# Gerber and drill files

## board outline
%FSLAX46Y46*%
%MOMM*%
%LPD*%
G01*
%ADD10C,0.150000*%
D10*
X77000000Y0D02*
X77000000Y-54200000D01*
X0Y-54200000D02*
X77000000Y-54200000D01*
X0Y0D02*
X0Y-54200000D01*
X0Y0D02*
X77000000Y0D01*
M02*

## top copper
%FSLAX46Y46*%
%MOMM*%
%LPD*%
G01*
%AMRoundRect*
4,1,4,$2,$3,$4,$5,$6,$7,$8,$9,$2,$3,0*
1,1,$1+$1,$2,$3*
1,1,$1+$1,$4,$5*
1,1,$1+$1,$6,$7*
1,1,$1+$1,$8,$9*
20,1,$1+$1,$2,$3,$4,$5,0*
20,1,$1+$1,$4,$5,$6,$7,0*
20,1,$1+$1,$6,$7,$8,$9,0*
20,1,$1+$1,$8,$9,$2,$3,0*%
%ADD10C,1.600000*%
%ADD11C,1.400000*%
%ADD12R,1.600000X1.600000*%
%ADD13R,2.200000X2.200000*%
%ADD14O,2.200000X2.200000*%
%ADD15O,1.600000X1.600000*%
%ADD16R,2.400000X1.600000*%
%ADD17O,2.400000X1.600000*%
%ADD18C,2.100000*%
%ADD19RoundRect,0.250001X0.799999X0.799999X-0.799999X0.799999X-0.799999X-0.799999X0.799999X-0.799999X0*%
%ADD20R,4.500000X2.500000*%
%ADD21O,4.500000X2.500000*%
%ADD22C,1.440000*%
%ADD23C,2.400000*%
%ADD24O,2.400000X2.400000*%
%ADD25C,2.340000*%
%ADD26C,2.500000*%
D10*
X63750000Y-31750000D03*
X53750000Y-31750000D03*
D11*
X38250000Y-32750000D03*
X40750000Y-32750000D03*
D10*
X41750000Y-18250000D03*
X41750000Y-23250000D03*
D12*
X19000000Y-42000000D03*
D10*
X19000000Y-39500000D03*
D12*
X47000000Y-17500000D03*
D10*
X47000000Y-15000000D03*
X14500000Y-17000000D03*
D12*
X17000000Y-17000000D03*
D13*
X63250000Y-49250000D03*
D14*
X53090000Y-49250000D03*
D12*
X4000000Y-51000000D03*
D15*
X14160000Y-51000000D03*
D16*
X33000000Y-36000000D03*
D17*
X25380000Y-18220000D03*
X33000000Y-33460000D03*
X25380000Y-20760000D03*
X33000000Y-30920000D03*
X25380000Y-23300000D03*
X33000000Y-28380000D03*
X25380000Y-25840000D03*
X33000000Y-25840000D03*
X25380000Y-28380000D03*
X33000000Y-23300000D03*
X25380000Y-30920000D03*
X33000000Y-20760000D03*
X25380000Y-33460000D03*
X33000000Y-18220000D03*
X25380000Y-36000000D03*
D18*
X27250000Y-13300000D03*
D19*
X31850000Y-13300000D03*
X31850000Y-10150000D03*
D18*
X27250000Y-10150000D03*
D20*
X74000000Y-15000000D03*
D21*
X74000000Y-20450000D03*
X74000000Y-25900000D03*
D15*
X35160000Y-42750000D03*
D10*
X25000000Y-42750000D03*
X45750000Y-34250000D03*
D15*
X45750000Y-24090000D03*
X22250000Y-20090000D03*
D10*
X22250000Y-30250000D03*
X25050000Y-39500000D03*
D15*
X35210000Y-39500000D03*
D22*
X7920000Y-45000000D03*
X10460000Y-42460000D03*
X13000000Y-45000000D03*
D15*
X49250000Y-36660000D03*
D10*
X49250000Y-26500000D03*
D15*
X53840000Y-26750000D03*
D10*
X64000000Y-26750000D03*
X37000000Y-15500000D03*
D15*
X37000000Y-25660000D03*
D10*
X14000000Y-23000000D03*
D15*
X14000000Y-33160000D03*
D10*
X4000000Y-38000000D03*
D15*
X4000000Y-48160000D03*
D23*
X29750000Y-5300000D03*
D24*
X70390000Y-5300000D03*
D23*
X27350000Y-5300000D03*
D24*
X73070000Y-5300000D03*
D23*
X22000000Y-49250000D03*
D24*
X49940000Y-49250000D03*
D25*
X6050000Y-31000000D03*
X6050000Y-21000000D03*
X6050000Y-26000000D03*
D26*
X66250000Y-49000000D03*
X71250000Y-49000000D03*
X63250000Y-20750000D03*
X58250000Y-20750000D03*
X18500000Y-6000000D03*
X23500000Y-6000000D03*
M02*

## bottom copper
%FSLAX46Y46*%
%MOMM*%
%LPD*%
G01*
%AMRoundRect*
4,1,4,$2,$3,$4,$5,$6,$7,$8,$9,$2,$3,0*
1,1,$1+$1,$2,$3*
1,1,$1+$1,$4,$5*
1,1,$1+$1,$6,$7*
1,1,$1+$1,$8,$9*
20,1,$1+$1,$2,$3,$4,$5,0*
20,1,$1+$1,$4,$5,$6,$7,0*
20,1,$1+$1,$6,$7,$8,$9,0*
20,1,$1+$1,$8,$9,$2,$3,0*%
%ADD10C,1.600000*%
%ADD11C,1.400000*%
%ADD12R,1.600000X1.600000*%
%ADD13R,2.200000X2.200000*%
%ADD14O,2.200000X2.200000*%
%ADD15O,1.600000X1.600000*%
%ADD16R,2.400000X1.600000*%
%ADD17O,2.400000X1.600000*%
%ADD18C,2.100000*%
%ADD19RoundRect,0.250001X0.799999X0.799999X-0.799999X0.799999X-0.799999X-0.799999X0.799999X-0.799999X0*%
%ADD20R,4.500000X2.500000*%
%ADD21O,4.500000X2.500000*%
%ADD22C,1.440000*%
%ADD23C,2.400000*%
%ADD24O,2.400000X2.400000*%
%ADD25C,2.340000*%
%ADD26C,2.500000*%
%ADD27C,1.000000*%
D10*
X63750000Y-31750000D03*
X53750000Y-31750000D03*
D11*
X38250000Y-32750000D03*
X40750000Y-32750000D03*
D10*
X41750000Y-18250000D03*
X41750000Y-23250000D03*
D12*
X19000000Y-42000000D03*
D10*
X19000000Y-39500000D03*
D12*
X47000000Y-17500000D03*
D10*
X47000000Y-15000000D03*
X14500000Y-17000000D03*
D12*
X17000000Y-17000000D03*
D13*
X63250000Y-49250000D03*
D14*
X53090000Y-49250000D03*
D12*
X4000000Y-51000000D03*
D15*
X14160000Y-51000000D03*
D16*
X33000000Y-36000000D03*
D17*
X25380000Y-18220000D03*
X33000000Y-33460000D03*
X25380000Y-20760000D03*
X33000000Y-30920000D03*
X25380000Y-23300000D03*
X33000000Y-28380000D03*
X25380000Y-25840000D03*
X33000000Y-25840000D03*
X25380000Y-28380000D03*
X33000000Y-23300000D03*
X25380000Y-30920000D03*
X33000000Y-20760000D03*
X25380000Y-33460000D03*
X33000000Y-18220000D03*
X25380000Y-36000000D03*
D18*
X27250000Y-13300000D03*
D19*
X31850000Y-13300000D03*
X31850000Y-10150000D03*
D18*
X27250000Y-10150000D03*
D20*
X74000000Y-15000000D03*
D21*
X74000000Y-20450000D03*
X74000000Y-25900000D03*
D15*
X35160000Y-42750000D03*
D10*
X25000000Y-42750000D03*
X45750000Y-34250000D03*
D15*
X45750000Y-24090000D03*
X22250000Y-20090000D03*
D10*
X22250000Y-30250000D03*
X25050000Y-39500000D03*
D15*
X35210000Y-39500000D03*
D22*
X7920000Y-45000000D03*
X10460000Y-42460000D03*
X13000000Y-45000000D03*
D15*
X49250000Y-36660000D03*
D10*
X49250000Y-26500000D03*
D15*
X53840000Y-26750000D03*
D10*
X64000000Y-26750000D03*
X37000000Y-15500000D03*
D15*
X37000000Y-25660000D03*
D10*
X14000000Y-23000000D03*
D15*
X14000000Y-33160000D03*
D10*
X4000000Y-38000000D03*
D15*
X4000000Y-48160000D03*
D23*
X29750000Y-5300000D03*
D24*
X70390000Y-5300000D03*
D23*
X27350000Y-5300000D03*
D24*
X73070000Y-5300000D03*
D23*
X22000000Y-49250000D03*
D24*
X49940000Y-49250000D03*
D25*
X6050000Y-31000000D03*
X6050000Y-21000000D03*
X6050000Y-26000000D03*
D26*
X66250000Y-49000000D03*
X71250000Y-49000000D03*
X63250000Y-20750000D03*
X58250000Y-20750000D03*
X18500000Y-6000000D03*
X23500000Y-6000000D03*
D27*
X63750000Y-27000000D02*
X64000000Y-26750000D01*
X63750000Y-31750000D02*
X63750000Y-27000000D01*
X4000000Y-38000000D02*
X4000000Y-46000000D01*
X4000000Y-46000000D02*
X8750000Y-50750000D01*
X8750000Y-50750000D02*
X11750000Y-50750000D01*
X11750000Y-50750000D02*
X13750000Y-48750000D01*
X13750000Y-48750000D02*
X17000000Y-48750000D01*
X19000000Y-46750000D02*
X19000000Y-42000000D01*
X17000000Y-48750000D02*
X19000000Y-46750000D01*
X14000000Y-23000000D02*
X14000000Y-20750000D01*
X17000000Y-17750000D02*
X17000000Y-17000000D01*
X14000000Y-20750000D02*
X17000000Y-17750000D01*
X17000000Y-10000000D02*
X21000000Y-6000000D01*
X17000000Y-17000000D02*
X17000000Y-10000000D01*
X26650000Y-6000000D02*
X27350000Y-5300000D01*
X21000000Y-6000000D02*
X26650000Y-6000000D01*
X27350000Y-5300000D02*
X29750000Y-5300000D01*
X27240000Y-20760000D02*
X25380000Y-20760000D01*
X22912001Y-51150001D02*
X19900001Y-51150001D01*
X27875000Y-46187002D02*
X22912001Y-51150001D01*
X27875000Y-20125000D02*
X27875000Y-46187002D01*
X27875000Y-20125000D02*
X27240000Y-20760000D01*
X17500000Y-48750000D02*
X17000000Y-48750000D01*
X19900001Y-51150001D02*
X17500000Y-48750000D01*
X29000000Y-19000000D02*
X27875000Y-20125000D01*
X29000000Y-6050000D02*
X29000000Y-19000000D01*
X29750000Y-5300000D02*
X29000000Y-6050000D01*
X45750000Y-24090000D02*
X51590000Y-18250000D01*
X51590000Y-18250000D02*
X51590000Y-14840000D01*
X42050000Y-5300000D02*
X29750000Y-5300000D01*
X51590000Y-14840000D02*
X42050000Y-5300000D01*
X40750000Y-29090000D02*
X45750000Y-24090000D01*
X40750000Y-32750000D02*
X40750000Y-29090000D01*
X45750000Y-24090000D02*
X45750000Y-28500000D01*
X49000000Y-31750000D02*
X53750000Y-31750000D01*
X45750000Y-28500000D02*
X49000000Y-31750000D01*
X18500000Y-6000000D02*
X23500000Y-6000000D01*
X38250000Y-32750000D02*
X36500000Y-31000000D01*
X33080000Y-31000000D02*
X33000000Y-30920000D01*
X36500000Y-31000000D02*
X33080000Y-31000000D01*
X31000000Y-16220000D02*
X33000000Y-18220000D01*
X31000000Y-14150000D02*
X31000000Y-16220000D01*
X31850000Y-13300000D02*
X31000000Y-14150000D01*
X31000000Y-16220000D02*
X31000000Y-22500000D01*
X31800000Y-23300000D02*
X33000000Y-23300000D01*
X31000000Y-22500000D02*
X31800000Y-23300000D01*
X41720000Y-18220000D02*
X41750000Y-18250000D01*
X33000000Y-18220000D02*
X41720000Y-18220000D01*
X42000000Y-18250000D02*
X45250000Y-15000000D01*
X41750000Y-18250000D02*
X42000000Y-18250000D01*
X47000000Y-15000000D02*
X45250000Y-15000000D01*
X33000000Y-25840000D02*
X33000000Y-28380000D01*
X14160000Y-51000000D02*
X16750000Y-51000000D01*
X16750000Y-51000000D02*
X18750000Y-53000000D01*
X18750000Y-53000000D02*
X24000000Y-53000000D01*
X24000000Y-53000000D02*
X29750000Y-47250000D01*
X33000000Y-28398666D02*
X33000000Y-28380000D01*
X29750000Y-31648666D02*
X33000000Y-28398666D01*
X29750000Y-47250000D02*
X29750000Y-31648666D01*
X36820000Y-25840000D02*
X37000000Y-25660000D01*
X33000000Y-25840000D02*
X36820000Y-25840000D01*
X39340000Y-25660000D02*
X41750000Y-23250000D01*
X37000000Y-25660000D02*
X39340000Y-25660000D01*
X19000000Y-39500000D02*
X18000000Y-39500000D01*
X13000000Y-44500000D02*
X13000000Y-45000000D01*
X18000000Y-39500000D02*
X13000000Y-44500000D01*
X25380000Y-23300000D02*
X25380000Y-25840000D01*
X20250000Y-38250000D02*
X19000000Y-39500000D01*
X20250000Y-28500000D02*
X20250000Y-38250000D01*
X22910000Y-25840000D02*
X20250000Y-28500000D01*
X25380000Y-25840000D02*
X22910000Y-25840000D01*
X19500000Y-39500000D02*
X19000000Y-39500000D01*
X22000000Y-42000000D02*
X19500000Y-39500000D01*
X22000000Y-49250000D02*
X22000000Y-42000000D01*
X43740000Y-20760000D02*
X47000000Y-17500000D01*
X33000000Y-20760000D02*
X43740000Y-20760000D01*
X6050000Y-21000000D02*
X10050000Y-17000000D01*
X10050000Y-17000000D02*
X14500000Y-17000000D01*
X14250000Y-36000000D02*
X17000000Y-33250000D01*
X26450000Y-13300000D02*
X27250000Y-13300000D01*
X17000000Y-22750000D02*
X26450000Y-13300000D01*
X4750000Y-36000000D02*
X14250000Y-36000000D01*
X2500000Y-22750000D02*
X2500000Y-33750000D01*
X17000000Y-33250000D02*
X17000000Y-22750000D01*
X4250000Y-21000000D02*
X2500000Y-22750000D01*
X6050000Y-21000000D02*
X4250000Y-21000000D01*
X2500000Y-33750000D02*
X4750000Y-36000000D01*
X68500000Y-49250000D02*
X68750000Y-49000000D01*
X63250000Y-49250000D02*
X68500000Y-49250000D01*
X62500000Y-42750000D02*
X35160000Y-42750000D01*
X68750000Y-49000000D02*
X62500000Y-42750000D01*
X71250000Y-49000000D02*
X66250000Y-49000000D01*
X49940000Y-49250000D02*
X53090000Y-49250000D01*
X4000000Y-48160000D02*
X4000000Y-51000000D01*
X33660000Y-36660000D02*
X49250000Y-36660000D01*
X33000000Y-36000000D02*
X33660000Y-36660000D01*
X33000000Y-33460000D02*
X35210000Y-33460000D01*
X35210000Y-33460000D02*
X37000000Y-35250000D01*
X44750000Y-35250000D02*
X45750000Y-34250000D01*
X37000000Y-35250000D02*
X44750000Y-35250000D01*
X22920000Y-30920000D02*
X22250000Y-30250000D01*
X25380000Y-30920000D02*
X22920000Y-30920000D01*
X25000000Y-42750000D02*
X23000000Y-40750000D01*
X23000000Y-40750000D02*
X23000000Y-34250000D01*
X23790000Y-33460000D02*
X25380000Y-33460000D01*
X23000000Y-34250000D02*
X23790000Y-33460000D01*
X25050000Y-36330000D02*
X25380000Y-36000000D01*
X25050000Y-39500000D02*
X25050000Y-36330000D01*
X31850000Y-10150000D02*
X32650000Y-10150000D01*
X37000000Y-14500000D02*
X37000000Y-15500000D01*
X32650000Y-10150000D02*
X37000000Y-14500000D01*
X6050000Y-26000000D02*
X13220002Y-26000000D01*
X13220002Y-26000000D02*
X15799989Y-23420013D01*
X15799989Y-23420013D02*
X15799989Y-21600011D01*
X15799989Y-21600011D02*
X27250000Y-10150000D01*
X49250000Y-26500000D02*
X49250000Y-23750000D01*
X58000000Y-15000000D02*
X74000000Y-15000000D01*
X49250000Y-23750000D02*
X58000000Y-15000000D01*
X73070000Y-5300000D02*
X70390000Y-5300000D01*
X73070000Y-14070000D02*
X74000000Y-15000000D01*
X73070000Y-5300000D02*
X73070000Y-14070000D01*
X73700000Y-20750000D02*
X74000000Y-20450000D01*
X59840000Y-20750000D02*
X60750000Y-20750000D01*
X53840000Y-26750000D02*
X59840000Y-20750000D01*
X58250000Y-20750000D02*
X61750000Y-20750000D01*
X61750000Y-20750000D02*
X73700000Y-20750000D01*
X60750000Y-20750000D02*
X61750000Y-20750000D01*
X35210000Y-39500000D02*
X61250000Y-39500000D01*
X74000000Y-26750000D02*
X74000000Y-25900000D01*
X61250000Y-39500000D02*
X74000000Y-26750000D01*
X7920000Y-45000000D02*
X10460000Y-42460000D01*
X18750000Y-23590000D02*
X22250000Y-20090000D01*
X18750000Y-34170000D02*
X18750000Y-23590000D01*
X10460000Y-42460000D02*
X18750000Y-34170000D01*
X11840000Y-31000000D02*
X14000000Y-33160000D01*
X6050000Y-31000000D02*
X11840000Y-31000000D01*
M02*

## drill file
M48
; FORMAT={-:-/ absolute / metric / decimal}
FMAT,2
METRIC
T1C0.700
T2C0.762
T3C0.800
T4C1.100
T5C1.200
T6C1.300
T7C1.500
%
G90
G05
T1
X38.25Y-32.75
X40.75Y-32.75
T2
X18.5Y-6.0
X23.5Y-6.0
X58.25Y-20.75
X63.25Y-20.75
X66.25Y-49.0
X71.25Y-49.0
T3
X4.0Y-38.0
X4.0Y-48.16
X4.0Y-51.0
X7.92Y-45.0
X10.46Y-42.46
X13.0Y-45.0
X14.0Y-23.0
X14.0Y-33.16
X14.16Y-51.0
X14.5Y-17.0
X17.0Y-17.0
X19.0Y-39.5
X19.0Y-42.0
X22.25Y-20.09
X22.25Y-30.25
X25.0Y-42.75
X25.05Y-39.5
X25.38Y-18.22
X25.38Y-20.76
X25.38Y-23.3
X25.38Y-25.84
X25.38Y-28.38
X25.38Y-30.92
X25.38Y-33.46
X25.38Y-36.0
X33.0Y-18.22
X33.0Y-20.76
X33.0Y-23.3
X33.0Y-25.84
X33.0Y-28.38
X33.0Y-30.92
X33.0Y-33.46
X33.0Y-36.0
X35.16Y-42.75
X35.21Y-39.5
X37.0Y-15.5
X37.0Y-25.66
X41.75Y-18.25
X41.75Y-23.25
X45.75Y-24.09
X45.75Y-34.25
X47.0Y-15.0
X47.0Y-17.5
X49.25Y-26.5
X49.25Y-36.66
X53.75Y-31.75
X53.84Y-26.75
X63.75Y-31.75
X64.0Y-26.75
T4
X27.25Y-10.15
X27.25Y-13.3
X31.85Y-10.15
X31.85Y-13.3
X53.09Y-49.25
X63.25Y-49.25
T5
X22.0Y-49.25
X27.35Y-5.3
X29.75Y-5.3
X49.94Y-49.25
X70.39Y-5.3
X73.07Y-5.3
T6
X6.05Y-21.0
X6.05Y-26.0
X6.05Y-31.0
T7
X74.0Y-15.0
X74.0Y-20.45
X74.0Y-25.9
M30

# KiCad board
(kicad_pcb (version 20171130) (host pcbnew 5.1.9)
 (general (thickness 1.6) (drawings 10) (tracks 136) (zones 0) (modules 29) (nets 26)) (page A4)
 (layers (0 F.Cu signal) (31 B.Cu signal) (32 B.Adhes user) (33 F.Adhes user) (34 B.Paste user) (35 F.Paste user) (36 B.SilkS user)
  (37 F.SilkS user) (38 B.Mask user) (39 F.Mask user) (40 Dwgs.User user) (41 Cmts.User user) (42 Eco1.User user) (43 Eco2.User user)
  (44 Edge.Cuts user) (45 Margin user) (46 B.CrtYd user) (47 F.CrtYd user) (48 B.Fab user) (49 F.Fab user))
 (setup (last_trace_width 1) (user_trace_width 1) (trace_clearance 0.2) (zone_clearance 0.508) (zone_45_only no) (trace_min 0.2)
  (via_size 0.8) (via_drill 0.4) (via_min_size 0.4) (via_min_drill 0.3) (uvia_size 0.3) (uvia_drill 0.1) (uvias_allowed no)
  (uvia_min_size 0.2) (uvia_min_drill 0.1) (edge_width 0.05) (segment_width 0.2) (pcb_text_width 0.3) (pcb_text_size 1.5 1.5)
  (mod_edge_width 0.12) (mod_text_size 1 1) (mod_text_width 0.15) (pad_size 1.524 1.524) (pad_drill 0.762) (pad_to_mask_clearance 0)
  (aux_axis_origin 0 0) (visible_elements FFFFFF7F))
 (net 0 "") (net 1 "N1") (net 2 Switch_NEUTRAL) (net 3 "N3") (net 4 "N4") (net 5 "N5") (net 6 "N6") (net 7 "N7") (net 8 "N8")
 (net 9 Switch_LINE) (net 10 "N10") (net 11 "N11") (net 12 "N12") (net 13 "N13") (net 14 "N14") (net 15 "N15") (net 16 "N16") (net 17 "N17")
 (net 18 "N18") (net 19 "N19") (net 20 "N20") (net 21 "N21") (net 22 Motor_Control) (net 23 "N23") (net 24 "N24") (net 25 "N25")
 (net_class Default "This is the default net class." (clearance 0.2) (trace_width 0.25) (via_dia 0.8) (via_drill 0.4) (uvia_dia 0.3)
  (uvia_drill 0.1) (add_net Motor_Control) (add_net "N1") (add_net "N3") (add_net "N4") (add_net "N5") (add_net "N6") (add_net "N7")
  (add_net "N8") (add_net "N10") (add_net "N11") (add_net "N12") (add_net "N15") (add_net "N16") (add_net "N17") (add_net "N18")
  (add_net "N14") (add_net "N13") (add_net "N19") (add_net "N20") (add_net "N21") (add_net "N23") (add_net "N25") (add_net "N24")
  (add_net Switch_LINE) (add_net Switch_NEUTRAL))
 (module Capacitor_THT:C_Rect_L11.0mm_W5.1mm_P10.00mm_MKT (layer F.Cu) (at 63.75 31.75 180)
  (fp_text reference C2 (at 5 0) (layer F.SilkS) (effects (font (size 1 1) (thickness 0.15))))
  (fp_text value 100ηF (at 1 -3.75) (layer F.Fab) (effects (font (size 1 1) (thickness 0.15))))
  (pad 1 thru_hole circle (at 0 0 180) (size 1.6 1.6) (drill 0.8) (layers *.Cu *.Mask) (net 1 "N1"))
  (pad 2 thru_hole circle (at 10 0 180) (size 1.6 1.6) (drill 0.8) (layers *.Cu *.Mask) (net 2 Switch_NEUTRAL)))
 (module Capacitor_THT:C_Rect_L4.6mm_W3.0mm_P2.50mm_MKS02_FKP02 (layer F.Cu) (at 38.25 32.75)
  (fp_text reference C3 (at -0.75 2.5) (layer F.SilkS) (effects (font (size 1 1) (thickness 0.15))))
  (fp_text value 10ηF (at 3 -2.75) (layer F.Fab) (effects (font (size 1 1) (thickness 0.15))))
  (pad 1 thru_hole circle (at 0 0) (size 1.4 1.4) (drill 0.7) (layers *.Cu *.Mask) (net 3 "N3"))
  (pad 2 thru_hole circle (at 2.5 0) (size 1.4 1.4) (drill 0.7) (layers *.Cu *.Mask) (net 2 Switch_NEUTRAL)))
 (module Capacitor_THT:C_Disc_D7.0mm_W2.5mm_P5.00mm (layer F.Cu) (at 41.75 18.25 270)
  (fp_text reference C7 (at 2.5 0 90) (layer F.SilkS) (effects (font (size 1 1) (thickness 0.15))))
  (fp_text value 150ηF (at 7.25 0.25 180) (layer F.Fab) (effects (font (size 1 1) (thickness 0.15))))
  (pad 1 thru_hole circle (at 0 0 270) (size 1.6 1.6) (drill 0.8) (layers *.Cu *.Mask) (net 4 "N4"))
  (pad 2 thru_hole circle (at 5 0 270) (size 1.6 1.6) (drill 0.8) (layers *.Cu *.Mask) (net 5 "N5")))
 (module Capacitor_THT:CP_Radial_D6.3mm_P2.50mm (layer F.Cu) (at 19 42 90)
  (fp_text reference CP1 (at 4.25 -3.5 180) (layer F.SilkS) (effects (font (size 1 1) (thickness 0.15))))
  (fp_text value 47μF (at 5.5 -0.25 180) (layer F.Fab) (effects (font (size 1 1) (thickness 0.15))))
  (pad 1 thru_hole rect (at 0 0 90) (size 1.6 1.6) (drill 0.8) (layers *.Cu *.Mask) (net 2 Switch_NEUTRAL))
  (pad 2 thru_hole circle (at 2.5 0 90) (size 1.6 1.6) (drill 0.8) (layers *.Cu *.Mask) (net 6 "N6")))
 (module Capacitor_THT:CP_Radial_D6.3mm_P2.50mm (layer F.Cu) (at 47 17.5 90)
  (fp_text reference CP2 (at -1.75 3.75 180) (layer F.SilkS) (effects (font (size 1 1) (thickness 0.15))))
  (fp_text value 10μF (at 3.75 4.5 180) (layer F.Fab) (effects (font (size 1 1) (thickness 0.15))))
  (pad 1 thru_hole rect (at 0 0 90) (size 1.6 1.6) (drill 0.8) (layers *.Cu *.Mask) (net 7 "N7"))
  (pad 2 thru_hole circle (at 2.5 0 90) (size 1.6 1.6) (drill 0.8) (layers *.Cu *.Mask) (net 4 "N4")))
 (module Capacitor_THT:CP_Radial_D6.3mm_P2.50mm (layer F.Cu) (at 17 17 180)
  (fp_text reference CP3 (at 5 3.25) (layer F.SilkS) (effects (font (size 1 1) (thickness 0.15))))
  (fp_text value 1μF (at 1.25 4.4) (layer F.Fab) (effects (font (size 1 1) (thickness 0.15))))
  (pad 2 thru_hole circle (at 2.5 0 180) (size 1.6 1.6) (drill 0.8) (layers *.Cu *.Mask) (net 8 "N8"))
  (pad 1 thru_hole rect (at 0 0 180) (size 1.6 1.6) (drill 0.8) (layers *.Cu *.Mask) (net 2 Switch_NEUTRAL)))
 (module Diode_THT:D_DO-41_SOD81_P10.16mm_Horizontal (layer F.Cu) (at 63.25 49.25 180)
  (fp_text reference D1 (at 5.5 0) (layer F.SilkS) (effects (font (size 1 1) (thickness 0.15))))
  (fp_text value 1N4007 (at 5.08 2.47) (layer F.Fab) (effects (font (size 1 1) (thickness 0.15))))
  (pad 1 thru_hole rect (at 0 0 180) (size 2.2 2.2) (drill 1.1) (layers *.Cu *.Mask) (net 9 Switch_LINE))
  (pad 2 thru_hole oval (at 10.16 0 180) (size 2.2 2.2) (drill 1.1) (layers *.Cu *.Mask) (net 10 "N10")))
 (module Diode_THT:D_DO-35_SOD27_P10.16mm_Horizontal (layer F.Cu) (at 4 51)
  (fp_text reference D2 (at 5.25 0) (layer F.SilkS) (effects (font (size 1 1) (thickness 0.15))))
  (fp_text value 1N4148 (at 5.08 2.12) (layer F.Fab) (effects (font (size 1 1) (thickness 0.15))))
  (pad 1 thru_hole rect (at 0 0) (size 1.6 1.6) (drill 0.8) (layers *.Cu *.Mask) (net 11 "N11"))
  (pad 2 thru_hole oval (at 10.16 0) (size 1.6 1.6) (drill 0.8) (layers *.Cu *.Mask) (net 5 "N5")))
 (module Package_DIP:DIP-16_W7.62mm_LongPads (layer F.Cu) (at 33 36 180)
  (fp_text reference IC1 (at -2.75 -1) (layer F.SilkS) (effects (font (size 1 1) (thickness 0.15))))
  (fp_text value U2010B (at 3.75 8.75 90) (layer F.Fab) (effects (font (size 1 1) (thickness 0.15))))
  (pad 1 thru_hole rect (at 0 0 180) (size 2.4 1.6) (drill 0.8) (layers *.Cu *.Mask) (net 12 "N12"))
  (pad 9 thru_hole oval (at 7.62 17.78 180) (size 2.4 1.6) (drill 0.8) (layers *.Cu *.Mask) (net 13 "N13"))
  (pad 2 thru_hole oval (at 0 2.54 180) (size 2.4 1.6) (drill 0.8) (layers *.Cu *.Mask) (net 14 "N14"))
  (pad 10 thru_hole oval (at 7.62 15.24 180) (size 2.4 1.6) (drill 0.8) (layers *.Cu *.Mask) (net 2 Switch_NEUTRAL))
  (pad 3 thru_hole oval (at 0 5.08 180) (size 2.4 1.6) (drill 0.8) (layers *.Cu *.Mask) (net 3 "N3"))
  (pad 11 thru_hole oval (at 7.62 12.7 180) (size 2.4 1.6) (drill 0.8) (layers *.Cu *.Mask) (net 6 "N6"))
  (pad 4 thru_hole oval (at 0 7.62 180) (size 2.4 1.6) (drill 0.8) (layers *.Cu *.Mask) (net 5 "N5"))
  (pad 12 thru_hole oval (at 7.62 10.16 180) (size 2.4 1.6) (drill 0.8) (layers *.Cu *.Mask) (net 6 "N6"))
  (pad 5 thru_hole oval (at 0 10.16 180) (size 2.4 1.6) (drill 0.8) (layers *.Cu *.Mask) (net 5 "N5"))
  (pad 13 thru_hole oval (at 7.62 7.62 180) (size 2.4 1.6) (drill 0.8) (layers *.Cu *.Mask) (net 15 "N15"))
  (pad 6 thru_hole oval (at 0 12.7 180) (size 2.4 1.6) (drill 0.8) (layers *.Cu *.Mask) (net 4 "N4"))
  (pad 14 thru_hole oval (at 7.62 5.08 180) (size 2.4 1.6) (drill 0.8) (layers *.Cu *.Mask) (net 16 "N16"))
  (pad 7 thru_hole oval (at 0 15.24 180) (size 2.4 1.6) (drill 0.8) (layers *.Cu *.Mask) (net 7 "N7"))
  (pad 15 thru_hole oval (at 7.62 2.54 180) (size 2.4 1.6) (drill 0.8) (layers *.Cu *.Mask) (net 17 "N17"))
  (pad 8 thru_hole oval (at 0 17.78 180) (size 2.4 1.6) (drill 0.8) (layers *.Cu *.Mask) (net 4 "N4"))
  (pad 16 thru_hole oval (at 7.62 0 180) (size 2.4 1.6) (drill 0.8) (layers *.Cu *.Mask) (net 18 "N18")))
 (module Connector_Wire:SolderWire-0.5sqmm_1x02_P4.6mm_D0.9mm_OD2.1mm (layer F.Cu) (at 31.85 13.3 180)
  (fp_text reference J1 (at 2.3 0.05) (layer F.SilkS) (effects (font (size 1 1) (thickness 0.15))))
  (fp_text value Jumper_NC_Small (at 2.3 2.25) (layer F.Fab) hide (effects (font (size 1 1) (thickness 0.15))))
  (pad 2 thru_hole circle (at 4.6 0 180) (size 2.1 2.1) (drill 1.1) (layers *.Cu *.Mask) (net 8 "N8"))
  (pad 1 thru_hole roundrect (at 0 0 180) (size 2.1 2.1) (drill 1.1) (layers *.Cu *.Mask) (roundrect_rratio 0.119048) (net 4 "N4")))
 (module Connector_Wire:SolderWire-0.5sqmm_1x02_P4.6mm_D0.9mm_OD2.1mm (layer F.Cu) (at 31.85 10.15 180)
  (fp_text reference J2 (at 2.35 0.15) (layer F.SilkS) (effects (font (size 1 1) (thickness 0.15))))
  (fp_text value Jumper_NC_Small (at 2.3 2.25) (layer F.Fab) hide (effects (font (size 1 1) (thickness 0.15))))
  (pad 1 thru_hole roundrect (at 0 0 180) (size 2.1 2.1) (drill 1.1) (layers *.Cu *.Mask) (roundrect_rratio 0.119048) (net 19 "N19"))
  (pad 2 thru_hole circle (at 4.6 0 180) (size 2.1 2.1) (drill 1.1) (layers *.Cu *.Mask) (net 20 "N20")))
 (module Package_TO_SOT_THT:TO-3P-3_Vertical (layer F.Cu) (at 74 15 270)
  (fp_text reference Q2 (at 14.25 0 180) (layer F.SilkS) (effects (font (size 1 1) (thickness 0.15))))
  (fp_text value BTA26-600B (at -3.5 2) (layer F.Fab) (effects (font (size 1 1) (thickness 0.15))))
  (pad 1 thru_hole rect (at 0 0 270) (size 2.5 4.5) (drill 1.5) (layers *.Cu *.Mask) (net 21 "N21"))
  (pad 2 thru_hole oval (at 5.45 0 270) (size 2.5 4.5) (drill 1.5) (layers *.Cu *.Mask) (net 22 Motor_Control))
  (pad 3 thru_hole oval (at 10.9 0 270) (size 2.5 4.5) (drill 1.5) (layers *.Cu *.Mask) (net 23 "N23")))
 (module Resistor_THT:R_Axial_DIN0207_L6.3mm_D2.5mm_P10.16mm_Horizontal (layer F.Cu) (at 25 42.75)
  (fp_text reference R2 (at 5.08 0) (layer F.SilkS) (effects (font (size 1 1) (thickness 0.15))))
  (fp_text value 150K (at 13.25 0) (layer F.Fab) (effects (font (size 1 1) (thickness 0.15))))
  (pad 2 thru_hole oval (at 10.16 0) (size 1.6 1.6) (drill 0.8) (layers *.Cu *.Mask) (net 9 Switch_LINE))
  (pad 1 thru_hole circle (at 0 0) (size 1.6 1.6) (drill 0.8) (layers *.Cu *.Mask) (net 17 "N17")))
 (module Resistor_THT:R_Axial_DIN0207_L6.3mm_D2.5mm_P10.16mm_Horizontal (layer F.Cu) (at 45.75 34.25 90)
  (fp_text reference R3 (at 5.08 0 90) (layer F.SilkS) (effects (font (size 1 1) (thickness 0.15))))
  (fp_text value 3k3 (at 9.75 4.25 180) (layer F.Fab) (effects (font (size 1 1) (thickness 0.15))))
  (pad 1 thru_hole circle (at 0 0 90) (size 1.6 1.6) (drill 0.8) (layers *.Cu *.Mask) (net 14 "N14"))
  (pad 2 thru_hole oval (at 10.16 0 90) (size 1.6 1.6) (drill 0.8) (layers *.Cu *.Mask) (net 2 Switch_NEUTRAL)))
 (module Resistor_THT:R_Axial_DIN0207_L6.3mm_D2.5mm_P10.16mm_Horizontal (layer F.Cu) (at 22.25 30.25 90)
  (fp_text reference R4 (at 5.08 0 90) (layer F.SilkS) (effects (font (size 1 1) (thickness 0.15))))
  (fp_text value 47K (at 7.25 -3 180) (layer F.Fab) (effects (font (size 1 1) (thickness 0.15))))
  (pad 2 thru_hole oval (at 10.16 0 90) (size 1.6 1.6) (drill 0.8) (layers *.Cu *.Mask) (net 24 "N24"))
  (pad 1 thru_hole circle (at 0 0 90) (size 1.6 1.6) (drill 0.8) (layers *.Cu *.Mask) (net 16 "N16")))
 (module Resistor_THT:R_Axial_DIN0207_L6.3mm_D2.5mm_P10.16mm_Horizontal (layer F.Cu) (at 25.05 39.5)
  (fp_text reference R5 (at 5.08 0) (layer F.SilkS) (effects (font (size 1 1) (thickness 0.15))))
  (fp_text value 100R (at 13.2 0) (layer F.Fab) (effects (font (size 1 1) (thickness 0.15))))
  (pad 1 thru_hole circle (at 0 0) (size 1.6 1.6) (drill 0.8) (layers *.Cu *.Mask) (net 18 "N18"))
  (pad 2 thru_hole oval (at 10.16 0) (size 1.6 1.6) (drill 0.8) (layers *.Cu *.Mask) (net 23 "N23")))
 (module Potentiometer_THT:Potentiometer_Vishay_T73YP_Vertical (layer F.Cu) (at 13 45 90)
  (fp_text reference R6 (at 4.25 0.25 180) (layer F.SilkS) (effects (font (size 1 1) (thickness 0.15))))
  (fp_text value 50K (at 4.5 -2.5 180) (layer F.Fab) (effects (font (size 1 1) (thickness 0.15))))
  (pad 3 thru_hole circle (at 0 -5.08 90) (size 1.44 1.44) (drill 0.8) (layers *.Cu *.Mask) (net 24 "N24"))
  (pad 2 thru_hole circle (at 2.54 -2.54 90) (size 1.44 1.44) (drill 0.8) (layers *.Cu *.Mask) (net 24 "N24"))
  (pad 1 thru_hole circle (at 0 0 90) (size 1.44 1.44) (drill 0.8) (layers *.Cu *.Mask) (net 6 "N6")))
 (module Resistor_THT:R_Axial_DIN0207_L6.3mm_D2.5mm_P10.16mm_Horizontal (layer F.Cu) (at 49.25 26.5 270)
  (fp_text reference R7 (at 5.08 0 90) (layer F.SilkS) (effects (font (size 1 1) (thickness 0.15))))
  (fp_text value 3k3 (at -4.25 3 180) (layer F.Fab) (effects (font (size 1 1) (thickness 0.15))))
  (pad 2 thru_hole oval (at 10.16 0 270) (size 1.6 1.6) (drill 0.8) (layers *.Cu *.Mask) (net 12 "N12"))
  (pad 1 thru_hole circle (at 0 0 270) (size 1.6 1.6) (drill 0.8) (layers *.Cu *.Mask) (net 21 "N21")))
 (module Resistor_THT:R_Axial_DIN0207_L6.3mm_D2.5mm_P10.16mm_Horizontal (layer F.Cu) (at 64 26.75 180)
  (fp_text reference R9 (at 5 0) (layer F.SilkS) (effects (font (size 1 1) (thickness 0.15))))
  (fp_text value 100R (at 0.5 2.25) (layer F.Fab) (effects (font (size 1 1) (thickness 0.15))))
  (pad 2 thru_hole oval (at 10.16 0 180) (size 1.6 1.6) (drill 0.8) (layers *.Cu *.Mask) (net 22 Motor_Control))
  (pad 1 thru_hole circle (at 0 0 180) (size 1.6 1.6) (drill 0.8) (layers *.Cu *.Mask) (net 1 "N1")))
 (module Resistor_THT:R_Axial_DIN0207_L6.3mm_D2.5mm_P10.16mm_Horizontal (layer F.Cu) (at 37 15.5 270)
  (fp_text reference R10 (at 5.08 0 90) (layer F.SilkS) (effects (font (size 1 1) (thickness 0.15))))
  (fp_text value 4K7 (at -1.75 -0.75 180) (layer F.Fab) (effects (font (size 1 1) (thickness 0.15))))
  (pad 1 thru_hole circle (at 0 0 270) (size 1.6 1.6) (drill 0.8) (layers *.Cu *.Mask) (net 19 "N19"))
  (pad 2 thru_hole oval (at 10.16 0 270) (size 1.6 1.6) (drill 0.8) (layers *.Cu *.Mask) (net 5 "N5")))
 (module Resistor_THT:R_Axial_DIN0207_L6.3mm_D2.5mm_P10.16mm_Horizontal (layer F.Cu) (at 14 23 270)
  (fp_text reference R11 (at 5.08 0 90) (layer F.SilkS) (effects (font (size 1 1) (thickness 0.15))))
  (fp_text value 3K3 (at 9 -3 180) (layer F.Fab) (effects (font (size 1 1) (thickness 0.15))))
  (pad 1 thru_hole circle (at 0 0 270) (size 1.6 1.6) (drill 0.8) (layers *.Cu *.Mask) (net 2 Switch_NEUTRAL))
  (pad 2 thru_hole oval (at 10.16 0 270) (size 1.6 1.6) (drill 0.8) (layers *.Cu *.Mask) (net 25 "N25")))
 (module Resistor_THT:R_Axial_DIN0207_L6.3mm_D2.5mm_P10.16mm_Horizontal (layer F.Cu) (at 4 38 270)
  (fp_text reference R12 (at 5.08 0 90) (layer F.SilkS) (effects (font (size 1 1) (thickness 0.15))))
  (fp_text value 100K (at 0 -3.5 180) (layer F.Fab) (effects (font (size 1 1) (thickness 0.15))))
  (pad 1 thru_hole circle (at 0 0 270) (size 1.6 1.6) (drill 0.8) (layers *.Cu *.Mask) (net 2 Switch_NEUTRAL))
  (pad 2 thru_hole oval (at 10.16 0 270) (size 1.6 1.6) (drill 0.8) (layers *.Cu *.Mask) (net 11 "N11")))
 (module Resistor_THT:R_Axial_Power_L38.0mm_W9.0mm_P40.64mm (layer F.Cu) (at 29.75 5.3)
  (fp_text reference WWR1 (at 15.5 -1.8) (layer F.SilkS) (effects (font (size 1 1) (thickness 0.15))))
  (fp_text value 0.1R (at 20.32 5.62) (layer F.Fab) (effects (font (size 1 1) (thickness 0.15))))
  (pad 1 thru_hole circle (at 0 0) (size 2.4 2.4) (drill 1.2) (layers *.Cu *.Mask) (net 2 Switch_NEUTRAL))
  (pad 2 thru_hole oval (at 40.64 0) (size 2.4 2.4) (drill 1.2) (layers *.Cu *.Mask) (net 21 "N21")))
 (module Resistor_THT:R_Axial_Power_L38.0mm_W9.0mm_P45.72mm (layer F.Cu) (at 27.35 5.3)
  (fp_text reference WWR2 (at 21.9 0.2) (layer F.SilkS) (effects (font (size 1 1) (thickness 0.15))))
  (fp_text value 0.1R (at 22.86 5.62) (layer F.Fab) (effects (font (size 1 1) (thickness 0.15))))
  (pad 1 thru_hole circle (at 0 0) (size 2.4 2.4) (drill 1.2) (layers *.Cu *.Mask) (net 2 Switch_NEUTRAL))
  (pad 2 thru_hole oval (at 45.72 0) (size 2.4 2.4) (drill 1.2) (layers *.Cu *.Mask) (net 21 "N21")))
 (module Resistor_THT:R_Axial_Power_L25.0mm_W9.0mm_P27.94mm (layer F.Cu) (at 22 49.25)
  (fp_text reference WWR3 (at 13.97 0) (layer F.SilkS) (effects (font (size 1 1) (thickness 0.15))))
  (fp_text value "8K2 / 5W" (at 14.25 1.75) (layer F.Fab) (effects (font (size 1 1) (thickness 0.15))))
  (pad 1 thru_hole circle (at 0 0) (size 2.4 2.4) (drill 1.2) (layers *.Cu *.Mask) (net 6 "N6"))
  (pad 2 thru_hole oval (at 27.94 0) (size 2.4 2.4) (drill 1.2) (layers *.Cu *.Mask) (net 10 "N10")))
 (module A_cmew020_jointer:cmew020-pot (layer F.Cu) (at 6.05 21 180)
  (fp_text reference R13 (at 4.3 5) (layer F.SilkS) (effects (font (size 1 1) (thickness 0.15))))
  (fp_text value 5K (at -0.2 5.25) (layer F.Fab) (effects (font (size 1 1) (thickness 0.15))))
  (pad 3 thru_hole circle (at 0 -10 180) (size 2.34 2.34) (drill 1.3) (layers *.Cu *.Mask) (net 25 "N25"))
  (pad 1 thru_hole circle (at 0 0 180) (size 2.34 2.34) (drill 1.3) (layers *.Cu *.Mask) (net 8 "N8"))
  (pad 2 thru_hole circle (at 0 -5 180) (size 2.34 2.34) (drill 1.3) (layers *.Cu *.Mask) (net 20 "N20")))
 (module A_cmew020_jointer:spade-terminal (layer F.Cu) (at 68.75 49)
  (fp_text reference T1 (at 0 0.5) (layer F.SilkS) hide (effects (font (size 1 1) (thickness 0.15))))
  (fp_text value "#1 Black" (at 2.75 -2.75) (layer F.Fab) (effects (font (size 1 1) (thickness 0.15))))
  (pad 1 thru_hole circle (at -2.5 0) (size 2.5 2.5) (drill 0.762) (layers *.Cu *.Mask) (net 9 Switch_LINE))
  (pad 1 thru_hole circle (at 2.5 0) (size 2.5 2.5) (drill 0.762) (layers *.Cu *.Mask) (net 9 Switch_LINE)))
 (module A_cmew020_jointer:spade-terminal (layer F.Cu) (at 60.75 20.75)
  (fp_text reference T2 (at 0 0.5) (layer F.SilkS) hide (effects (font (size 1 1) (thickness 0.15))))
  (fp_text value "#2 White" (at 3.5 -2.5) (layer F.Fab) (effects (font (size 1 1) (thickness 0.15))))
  (pad 1 thru_hole circle (at 2.5 0) (size 2.5 2.5) (drill 0.762) (layers *.Cu *.Mask) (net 22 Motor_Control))
  (pad 1 thru_hole circle (at -2.5 0) (size 2.5 2.5) (drill 0.762) (layers *.Cu *.Mask) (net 22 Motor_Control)))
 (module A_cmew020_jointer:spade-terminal (layer F.Cu) (at 21 6)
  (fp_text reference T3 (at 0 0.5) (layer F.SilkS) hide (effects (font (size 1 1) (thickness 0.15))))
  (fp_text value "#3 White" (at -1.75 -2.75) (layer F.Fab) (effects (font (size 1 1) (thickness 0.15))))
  (pad 1 thru_hole circle (at -2.5 0) (size 2.5 2.5) (drill 0.762) (layers *.Cu *.Mask) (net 2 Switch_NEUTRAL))
  (pad 1 thru_hole circle (at 2.5 0) (size 2.5 2.5) (drill 0.762) (layers *.Cu *.Mask) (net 2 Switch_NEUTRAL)))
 (gr_line (start 77 0) (end 77 54.2) (layer Edge.Cuts) (width 0.15))
 (gr_line (start 0 54.2) (end 77 54.2) (layer Edge.Cuts) (width 0.15))
 (gr_line (start 0 0) (end 0 54.2) (layer Edge.Cuts) (width 0.15))
 (gr_line (start 0 0) (end 77 0) (layer Edge.Cuts) (width 0.15))
 (segment (start 63.75 27) (end 64 26.75) (width 1) (layer B.Cu) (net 1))
 (segment (start 63.75 31.75) (end 63.75 27) (width 1) (layer B.Cu) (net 1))
 (segment (start 4 38) (end 4 46) (width 1) (layer B.Cu) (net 2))
 (segment (start 4 46) (end 8.75 50.75) (width 1) (layer B.Cu) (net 2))
 (segment (start 8.75 50.75) (end 11.75 50.75) (width 1) (layer B.Cu) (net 2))
 (segment (start 11.75 50.75) (end 13.75 48.75) (width 1) (layer B.Cu) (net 2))
 (segment (start 13.75 48.75) (end 17 48.75) (width 1) (layer B.Cu) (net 2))
 (segment (start 19 46.75) (end 19 42) (width 1) (layer B.Cu) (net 2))
 (segment (start 17 48.75) (end 19 46.75) (width 1) (layer B.Cu) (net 2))
 (segment (start 14 23) (end 14 20.75) (width 1) (layer B.Cu) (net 2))
 (segment (start 17 17.75) (end 17 17) (width 1) (layer B.Cu) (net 2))
 (segment (start 14 20.75) (end 17 17.75) (width 1) (layer B.Cu) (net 2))
 (segment (start 17 10) (end 21 6) (width 1) (layer B.Cu) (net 2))
 (segment (start 17 17) (end 17 10) (width 1) (layer B.Cu) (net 2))
 (segment (start 26.65 6) (end 27.35 5.3) (width 1) (layer B.Cu) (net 2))
 (segment (start 21 6) (end 26.65 6) (width 1) (layer B.Cu) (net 2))
 (segment (start 27.35 5.3) (end 29.75 5.3) (width 1) (layer B.Cu) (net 2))
 (segment (start 27.24 20.76) (end 25.38 20.76) (width 1) (layer B.Cu) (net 2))
 (segment (start 22.912001 51.150001) (end 19.900001 51.150001) (width 1) (layer B.Cu) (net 2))
 (segment (start 27.875 46.187002) (end 22.912001 51.150001) (width 1) (layer B.Cu) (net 2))
 (segment (start 27.875 20.125) (end 27.875 46.187002) (width 1) (layer B.Cu) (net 2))
 (segment (start 27.875 20.125) (end 27.24 20.76) (width 1) (layer B.Cu) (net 2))
 (segment (start 17.5 48.75) (end 17 48.75) (width 1) (layer B.Cu) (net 2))
 (segment (start 19.900001 51.150001) (end 17.5 48.75) (width 1) (layer B.Cu) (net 2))
 (segment (start 29 19) (end 27.875 20.125) (width 1) (layer B.Cu) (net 2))
 (segment (start 29 6.05) (end 29 19) (width 1) (layer B.Cu) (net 2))
 (segment (start 29.75 5.3) (end 29 6.05) (width 1) (layer B.Cu) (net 2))
 (segment (start 45.75 24.09) (end 51.59 18.25) (width 1) (layer B.Cu) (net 2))
 (segment (start 51.59 18.25) (end 51.59 14.84) (width 1) (layer B.Cu) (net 2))
 (segment (start 42.05 5.3) (end 29.75 5.3) (width 1) (layer B.Cu) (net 2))
 (segment (start 51.59 14.84) (end 42.05 5.3) (width 1) (layer B.Cu) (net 2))
 (segment (start 40.75 29.09) (end 45.75 24.09) (width 1) (layer B.Cu) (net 2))
 (segment (start 40.75 32.75) (end 40.75 29.09) (width 1) (layer B.Cu) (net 2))
 (segment (start 45.75 24.09) (end 45.75 28.5) (width 1) (layer B.Cu) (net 2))
 (segment (start 49 31.75) (end 53.75 31.75) (width 1) (layer B.Cu) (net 2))
 (segment (start 45.75 28.5) (end 49 31.75) (width 1) (layer B.Cu) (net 2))
 (segment (start 18.5 6) (end 23.5 6) (width 1) (layer B.Cu) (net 2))
 (segment (start 38.25 32.75) (end 36.5 31) (width 1) (layer B.Cu) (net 3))
 (segment (start 33.08 31) (end 33 30.92) (width 1) (layer B.Cu) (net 3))
 (segment (start 36.5 31) (end 33.08 31) (width 1) (layer B.Cu) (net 3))
 (segment (start 31 16.22) (end 33 18.22) (width 1) (layer B.Cu) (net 4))
 (segment (start 31 14.15) (end 31 16.22) (width 1) (layer B.Cu) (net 4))
 (segment (start 31.85 13.3) (end 31 14.15) (width 1) (layer B.Cu) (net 4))
 (segment (start 31 16.22) (end 31 22.5) (width 1) (layer B.Cu) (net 4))
 (segment (start 31.8 23.3) (end 33 23.3) (width 1) (layer B.Cu) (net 4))
 (segment (start 31 22.5) (end 31.8 23.3) (width 1) (layer B.Cu) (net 4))
 (segment (start 41.72 18.22) (end 41.75 18.25) (width 1) (layer B.Cu) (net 4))
 (segment (start 33 18.22) (end 41.72 18.22) (width 1) (layer B.Cu) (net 4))
 (segment (start 42 18.25) (end 45.25 15) (width 1) (layer B.Cu) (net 4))
 (segment (start 41.75 18.25) (end 42 18.25) (width 1) (layer B.Cu) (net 4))
 (segment (start 47 15) (end 45.25 15) (width 1) (layer B.Cu) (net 4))
 (segment (start 33 25.84) (end 33 28.38) (width 1) (layer B.Cu) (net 5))
 (segment (start 14.16 51) (end 16.75 51) (width 1) (layer B.Cu) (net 5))
 (segment (start 16.75 51) (end 18.75 53) (width 1) (layer B.Cu) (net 5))
 (segment (start 18.75 53) (end 24 53) (width 1) (layer B.Cu) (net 5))
 (segment (start 24 53) (end 29.75 47.25) (width 1) (layer B.Cu) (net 5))
 (segment (start 33 28.398666) (end 33 28.38) (width 1) (layer B.Cu) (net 5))
 (segment (start 29.75 31.648666) (end 33 28.398666) (width 1) (layer B.Cu) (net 5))
 (segment (start 29.75 47.25) (end 29.75 31.648666) (width 1) (layer B.Cu) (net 5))
 (segment (start 36.82 25.84) (end 37 25.66) (width 1) (layer B.Cu) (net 5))
 (segment (start 33 25.84) (end 36.82 25.84) (width 1) (layer B.Cu) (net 5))
 (segment (start 39.34 25.66) (end 41.75 23.25) (width 1) (layer B.Cu) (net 5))
 (segment (start 37 25.66) (end 39.34 25.66) (width 1) (layer B.Cu) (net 5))
 (segment (start 19 39.5) (end 18 39.5) (width 1) (layer B.Cu) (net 6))
 (segment (start 13 44.5) (end 13 45) (width 1) (layer B.Cu) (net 6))
 (segment (start 18 39.5) (end 13 44.5) (width 1) (layer B.Cu) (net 6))
 (segment (start 25.38 23.3) (end 25.38 25.84) (width 1) (layer B.Cu) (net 6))
 (segment (start 20.25 38.25) (end 19 39.5) (width 1) (layer B.Cu) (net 6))
 (segment (start 20.25 28.5) (end 20.25 38.25) (width 1) (layer B.Cu) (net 6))
 (segment (start 22.91 25.84) (end 20.25 28.5) (width 1) (layer B.Cu) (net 6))
 (segment (start 25.38 25.84) (end 22.91 25.84) (width 1) (layer B.Cu) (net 6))
 (segment (start 19.5 39.5) (end 19 39.5) (width 1) (layer B.Cu) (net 6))
 (segment (start 22 42) (end 19.5 39.5) (width 1) (layer B.Cu) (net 6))
 (segment (start 22 49.25) (end 22 42) (width 1) (layer B.Cu) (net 6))
 (segment (start 43.74 20.76) (end 47 17.5) (width 1) (layer B.Cu) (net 7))
 (segment (start 33 20.76) (end 43.74 20.76) (width 1) (layer B.Cu) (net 7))
 (segment (start 6.05 21) (end 10.05 17) (width 1) (layer B.Cu) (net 8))
 (segment (start 10.05 17) (end 14.5 17) (width 1) (layer B.Cu) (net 8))
 (segment (start 14.25 36) (end 17 33.25) (width 1) (layer B.Cu) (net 8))
 (segment (start 26.45 13.3) (end 27.25 13.3) (width 1) (layer B.Cu) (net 8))
 (segment (start 17 22.75) (end 26.45 13.3) (width 1) (layer B.Cu) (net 8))
 (segment (start 4.75 36) (end 14.25 36) (width 1) (layer B.Cu) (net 8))
 (segment (start 2.5 22.75) (end 2.5 33.75) (width 1) (layer B.Cu) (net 8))
 (segment (start 17 33.25) (end 17 22.75) (width 1) (layer B.Cu) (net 8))
 (segment (start 4.25 21) (end 2.5 22.75) (width 1) (layer B.Cu) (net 8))
 (segment (start 6.05 21) (end 4.25 21) (width 1) (layer B.Cu) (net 8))
 (segment (start 2.5 33.75) (end 4.75 36) (width 1) (layer B.Cu) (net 8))
 (segment (start 68.5 49.25) (end 68.75 49) (width 1) (layer B.Cu) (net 9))
 (segment (start 63.25 49.25) (end 68.5 49.25) (width 1) (layer B.Cu) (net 9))
 (segment (start 62.5 42.75) (end 35.16 42.75) (width 1) (layer B.Cu) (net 9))
 (segment (start 68.75 49) (end 62.5 42.75) (width 1) (layer B.Cu) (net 9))
 (segment (start 71.25 49) (end 66.25 49) (width 1) (layer B.Cu) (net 9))
 (segment (start 49.94 49.25) (end 53.09 49.25) (width 1) (layer B.Cu) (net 10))
 (segment (start 4 48.16) (end 4 51) (width 1) (layer B.Cu) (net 11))
 (segment (start 33.66 36.66) (end 49.25 36.66) (width 1) (layer B.Cu) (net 12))
 (segment (start 33 36) (end 33.66 36.66) (width 1) (layer B.Cu) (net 12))
 (segment (start 33 33.46) (end 35.21 33.46) (width 1) (layer B.Cu) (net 14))
 (segment (start 35.21 33.46) (end 37 35.25) (width 1) (layer B.Cu) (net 14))
 (segment (start 44.75 35.25) (end 45.75 34.25) (width 1) (layer B.Cu) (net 14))
 (segment (start 37 35.25) (end 44.75 35.25) (width 1) (layer B.Cu) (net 14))
 (segment (start 22.92 30.92) (end 22.25 30.25) (width 1) (layer B.Cu) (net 16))
 (segment (start 25.38 30.92) (end 22.92 30.92) (width 1) (layer B.Cu) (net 16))
 (segment (start 25 42.75) (end 23 40.75) (width 1) (layer B.Cu) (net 17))
 (segment (start 23 40.75) (end 23 34.25) (width 1) (layer B.Cu) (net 17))
 (segment (start 23.79 33.46) (end 25.38 33.46) (width 1) (layer B.Cu) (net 17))
 (segment (start 23 34.25) (end 23.79 33.46) (width 1) (layer B.Cu) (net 17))
 (segment (start 25.05 36.33) (end 25.38 36) (width 1) (layer B.Cu) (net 18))
 (segment (start 25.05 39.5) (end 25.05 36.33) (width 1) (layer B.Cu) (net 18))
 (segment (start 31.85 10.15) (end 32.65 10.15) (width 1) (layer B.Cu) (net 19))
 (segment (start 37 14.5) (end 37 15.5) (width 1) (layer B.Cu) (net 19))
 (segment (start 32.65 10.15) (end 37 14.5) (width 1) (layer B.Cu) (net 19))
 (segment (start 6.05 26) (end 13.220002 26) (width 1) (layer B.Cu) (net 20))
 (segment (start 13.220002 26) (end 15.799989 23.420013) (width 1) (layer B.Cu) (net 20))
 (segment (start 15.799989 23.420013) (end 15.799989 21.600011) (width 1) (layer B.Cu) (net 20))
 (segment (start 15.799989 21.600011) (end 27.25 10.15) (width 1) (layer B.Cu) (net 20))
 (segment (start 49.25 26.5) (end 49.25 23.75) (width 1) (layer B.Cu) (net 21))
 (segment (start 58 15) (end 74 15) (width 1) (layer B.Cu) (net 21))
 (segment (start 49.25 23.75) (end 58 15) (width 1) (layer B.Cu) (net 21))
 (segment (start 73.07 5.3) (end 70.39 5.3) (width 1) (layer B.Cu) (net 21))
 (segment (start 73.07 14.07) (end 74 15) (width 1) (layer B.Cu) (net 21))
 (segment (start 73.07 5.3) (end 73.07 14.07) (width 1) (layer B.Cu) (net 21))
 (segment (start 73.7 20.75) (end 74 20.45) (width 1) (layer B.Cu) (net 22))
 (segment (start 59.84 20.75) (end 60.75 20.75) (width 1) (layer B.Cu) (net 22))
 (segment (start 53.84 26.75) (end 59.84 20.75) (width 1) (layer B.Cu) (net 22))
 (segment (start 58.25 20.75) (end 61.75 20.75) (width 1) (layer B.Cu) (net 22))
 (segment (start 61.75 20.75) (end 73.7 20.75) (width 1) (layer B.Cu) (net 22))
 (segment (start 60.75 20.75) (end 61.75 20.75) (width 1) (layer B.Cu) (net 22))
 (segment (start 35.21 39.5) (end 61.25 39.5) (width 1) (layer B.Cu) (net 23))
 (segment (start 74 26.75) (end 74 25.9) (width 1) (layer B.Cu) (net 23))
 (segment (start 61.25 39.5) (end 74 26.75) (width 1) (layer B.Cu) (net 23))
 (segment (start 7.92 45) (end 10.46 42.46) (width 1) (layer B.Cu) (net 24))
 (segment (start 18.75 23.59) (end 22.25 20.09) (width 1) (layer B.Cu) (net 24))
 (segment (start 18.75 34.17) (end 18.75 23.59) (width 1) (layer B.Cu) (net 24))
 (segment (start 10.46 42.46) (end 18.75 34.17) (width 1) (layer B.Cu) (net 24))
 (segment (start 11.84 31) (end 14 33.16) (width 1) (layer B.Cu) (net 25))
 (segment (start 6.05 31) (end 11.84 31) (width 1) (layer B.Cu) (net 25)))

